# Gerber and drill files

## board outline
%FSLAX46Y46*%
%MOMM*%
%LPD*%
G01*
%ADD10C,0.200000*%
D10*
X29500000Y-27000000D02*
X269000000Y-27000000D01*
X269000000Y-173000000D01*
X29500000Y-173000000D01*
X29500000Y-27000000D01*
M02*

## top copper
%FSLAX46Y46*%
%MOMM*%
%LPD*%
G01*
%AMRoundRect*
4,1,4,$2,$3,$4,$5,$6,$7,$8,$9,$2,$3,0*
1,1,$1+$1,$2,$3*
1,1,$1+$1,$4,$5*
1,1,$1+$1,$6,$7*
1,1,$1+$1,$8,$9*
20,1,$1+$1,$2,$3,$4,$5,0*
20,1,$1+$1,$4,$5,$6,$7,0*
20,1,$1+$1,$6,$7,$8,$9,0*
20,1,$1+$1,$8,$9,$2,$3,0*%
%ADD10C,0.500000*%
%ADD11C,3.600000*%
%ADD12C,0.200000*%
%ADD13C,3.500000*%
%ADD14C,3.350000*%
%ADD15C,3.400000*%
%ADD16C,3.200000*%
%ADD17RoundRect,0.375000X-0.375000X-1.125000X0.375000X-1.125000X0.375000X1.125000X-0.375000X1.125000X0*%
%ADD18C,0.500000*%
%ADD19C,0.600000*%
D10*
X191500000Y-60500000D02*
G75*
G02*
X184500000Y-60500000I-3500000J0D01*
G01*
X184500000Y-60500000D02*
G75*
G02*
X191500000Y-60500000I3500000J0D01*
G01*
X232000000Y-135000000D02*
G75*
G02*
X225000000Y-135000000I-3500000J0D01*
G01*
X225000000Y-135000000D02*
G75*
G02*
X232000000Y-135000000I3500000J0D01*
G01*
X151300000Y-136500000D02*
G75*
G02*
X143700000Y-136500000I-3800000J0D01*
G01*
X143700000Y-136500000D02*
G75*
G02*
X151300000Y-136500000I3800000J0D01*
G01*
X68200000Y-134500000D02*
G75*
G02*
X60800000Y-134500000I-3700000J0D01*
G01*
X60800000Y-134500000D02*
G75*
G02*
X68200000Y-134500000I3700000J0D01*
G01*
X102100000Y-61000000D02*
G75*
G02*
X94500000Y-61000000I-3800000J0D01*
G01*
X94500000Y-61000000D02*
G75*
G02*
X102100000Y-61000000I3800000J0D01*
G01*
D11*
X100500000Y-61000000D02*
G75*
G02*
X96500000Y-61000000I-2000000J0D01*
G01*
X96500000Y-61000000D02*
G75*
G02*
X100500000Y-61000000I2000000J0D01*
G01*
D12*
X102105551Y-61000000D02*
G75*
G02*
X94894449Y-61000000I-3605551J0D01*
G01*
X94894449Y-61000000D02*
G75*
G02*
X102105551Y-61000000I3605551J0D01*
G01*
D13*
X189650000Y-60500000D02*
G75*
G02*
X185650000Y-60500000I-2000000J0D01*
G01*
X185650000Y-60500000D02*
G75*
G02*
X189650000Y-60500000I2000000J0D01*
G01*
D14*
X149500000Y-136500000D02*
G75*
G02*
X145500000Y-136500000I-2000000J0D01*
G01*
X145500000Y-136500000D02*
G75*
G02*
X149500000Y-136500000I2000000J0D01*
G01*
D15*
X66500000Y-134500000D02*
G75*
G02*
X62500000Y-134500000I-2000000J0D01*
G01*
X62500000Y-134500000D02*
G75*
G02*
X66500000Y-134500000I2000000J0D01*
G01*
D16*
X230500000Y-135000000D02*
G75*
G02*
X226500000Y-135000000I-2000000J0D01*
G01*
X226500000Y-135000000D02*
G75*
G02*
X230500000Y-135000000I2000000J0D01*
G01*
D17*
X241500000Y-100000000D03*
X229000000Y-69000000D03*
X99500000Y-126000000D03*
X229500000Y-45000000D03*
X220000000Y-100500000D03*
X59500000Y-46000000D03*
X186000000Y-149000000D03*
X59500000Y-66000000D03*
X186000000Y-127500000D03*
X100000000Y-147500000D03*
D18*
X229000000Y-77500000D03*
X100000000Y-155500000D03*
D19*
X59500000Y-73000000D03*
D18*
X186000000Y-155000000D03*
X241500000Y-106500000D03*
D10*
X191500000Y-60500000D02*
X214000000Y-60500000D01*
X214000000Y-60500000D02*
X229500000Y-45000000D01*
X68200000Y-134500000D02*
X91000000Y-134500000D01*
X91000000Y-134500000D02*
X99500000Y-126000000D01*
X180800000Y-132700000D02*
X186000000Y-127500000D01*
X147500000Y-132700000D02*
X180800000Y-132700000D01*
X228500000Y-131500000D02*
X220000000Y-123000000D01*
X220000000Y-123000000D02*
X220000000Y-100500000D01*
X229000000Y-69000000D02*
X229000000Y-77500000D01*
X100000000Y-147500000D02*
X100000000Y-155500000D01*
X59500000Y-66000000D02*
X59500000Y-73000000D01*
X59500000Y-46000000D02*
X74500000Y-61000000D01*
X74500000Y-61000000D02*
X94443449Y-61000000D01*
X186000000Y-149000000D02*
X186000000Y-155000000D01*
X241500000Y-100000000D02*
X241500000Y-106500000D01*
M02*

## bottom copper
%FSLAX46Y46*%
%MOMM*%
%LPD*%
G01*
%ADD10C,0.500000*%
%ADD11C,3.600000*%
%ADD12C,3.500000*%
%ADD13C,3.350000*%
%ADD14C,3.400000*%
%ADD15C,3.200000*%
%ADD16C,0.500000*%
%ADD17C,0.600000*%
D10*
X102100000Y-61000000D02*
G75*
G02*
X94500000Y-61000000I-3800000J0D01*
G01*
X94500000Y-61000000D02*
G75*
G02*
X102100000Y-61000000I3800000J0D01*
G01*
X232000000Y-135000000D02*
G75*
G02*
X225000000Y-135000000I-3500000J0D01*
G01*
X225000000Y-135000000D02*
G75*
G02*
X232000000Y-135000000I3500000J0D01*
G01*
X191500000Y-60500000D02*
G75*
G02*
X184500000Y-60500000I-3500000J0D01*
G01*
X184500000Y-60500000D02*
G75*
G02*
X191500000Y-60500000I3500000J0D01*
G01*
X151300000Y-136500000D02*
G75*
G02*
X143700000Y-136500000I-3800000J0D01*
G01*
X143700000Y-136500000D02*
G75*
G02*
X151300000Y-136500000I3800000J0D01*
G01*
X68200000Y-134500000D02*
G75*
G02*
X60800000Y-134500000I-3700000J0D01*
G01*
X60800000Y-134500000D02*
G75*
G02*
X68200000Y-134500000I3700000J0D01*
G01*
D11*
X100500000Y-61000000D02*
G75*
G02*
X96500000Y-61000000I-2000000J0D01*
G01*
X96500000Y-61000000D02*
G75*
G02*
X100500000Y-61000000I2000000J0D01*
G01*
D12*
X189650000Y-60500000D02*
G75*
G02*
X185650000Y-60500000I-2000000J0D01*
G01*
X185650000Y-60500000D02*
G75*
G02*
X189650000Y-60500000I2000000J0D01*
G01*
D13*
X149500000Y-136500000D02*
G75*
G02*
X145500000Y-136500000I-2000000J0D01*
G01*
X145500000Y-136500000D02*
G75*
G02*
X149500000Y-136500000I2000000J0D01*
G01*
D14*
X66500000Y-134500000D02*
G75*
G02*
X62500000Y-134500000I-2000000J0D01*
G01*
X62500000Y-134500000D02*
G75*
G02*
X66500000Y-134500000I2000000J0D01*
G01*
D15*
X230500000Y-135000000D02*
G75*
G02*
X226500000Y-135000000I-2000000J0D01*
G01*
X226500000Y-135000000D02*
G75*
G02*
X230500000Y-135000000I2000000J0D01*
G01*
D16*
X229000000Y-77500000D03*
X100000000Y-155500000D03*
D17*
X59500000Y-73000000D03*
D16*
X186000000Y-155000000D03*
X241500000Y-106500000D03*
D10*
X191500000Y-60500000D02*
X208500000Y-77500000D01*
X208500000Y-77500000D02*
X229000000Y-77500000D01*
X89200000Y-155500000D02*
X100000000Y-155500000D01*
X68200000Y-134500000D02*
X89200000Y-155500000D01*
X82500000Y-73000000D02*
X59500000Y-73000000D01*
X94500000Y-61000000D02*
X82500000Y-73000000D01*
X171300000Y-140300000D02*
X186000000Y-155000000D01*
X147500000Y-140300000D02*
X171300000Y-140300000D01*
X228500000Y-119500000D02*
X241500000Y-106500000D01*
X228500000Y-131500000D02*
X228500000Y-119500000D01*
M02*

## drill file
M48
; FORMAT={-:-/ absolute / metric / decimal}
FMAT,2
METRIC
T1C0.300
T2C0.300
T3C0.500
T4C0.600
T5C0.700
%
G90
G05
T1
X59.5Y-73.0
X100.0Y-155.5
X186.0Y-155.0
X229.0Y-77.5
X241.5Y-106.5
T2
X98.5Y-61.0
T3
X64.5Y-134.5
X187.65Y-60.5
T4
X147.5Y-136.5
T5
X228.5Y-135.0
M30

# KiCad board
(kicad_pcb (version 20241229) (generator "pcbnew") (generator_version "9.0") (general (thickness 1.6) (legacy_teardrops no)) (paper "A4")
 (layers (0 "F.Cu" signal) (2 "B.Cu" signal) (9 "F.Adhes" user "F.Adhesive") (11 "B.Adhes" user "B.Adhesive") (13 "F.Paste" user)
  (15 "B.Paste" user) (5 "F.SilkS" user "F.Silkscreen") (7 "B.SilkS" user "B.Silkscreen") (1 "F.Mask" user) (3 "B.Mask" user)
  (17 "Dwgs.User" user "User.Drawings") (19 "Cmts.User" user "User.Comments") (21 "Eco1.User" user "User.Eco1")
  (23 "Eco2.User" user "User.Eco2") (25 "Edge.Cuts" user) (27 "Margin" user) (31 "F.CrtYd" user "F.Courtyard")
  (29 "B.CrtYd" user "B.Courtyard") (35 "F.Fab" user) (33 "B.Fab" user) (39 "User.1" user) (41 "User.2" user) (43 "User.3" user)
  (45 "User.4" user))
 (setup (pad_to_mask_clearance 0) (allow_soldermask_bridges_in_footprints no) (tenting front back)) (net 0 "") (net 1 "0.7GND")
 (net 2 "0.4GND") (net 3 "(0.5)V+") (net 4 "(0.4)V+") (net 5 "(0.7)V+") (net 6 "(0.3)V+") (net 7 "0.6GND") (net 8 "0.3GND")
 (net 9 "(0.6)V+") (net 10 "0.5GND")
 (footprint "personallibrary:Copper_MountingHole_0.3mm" (layer "F.Cu") (at 98.5 61.5)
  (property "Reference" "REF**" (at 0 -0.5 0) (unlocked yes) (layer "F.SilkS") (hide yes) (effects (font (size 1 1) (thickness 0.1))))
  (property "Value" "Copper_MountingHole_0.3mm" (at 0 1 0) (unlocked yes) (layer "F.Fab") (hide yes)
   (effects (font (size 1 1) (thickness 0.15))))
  (fp_circle (center 0 -0.5) (end 2 -0.5) (stroke (width 3.6) (type solid)) (fill no) (layers "F.Cu" "F.Mask"))
  (fp_circle (center 0 -0.5) (end 3 -2.5) (stroke (width 0.2) (type solid)) (fill no) (layer "F.Cu"))
  (fp_circle (center 0 -0.5) (end 2 -0.5) (stroke (width 3.6) (type solid)) (fill no) (layers "B.Cu" "B.Mask"))
  (pad "" np_thru_hole circle (at 0 -0.5) (size 0.3 0.3) (drill 0.3) (layers "*.Cu" "*.Mask")))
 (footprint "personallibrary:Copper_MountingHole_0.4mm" (layer "F.Cu") (at 187.5 60.5)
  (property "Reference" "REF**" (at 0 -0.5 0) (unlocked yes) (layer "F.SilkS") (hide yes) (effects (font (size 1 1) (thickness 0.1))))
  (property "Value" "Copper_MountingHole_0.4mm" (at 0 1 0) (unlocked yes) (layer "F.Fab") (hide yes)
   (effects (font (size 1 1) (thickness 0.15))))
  (fp_circle (center 0.15 0) (end 2.15 0) (stroke (width 3.5) (type solid)) (fill no) (layers "F.Cu" "F.Mask"))
  (fp_circle (center 0.15 0) (end 2.15 0) (stroke (width 3.5) (type solid)) (fill no) (layers "B.Cu" "B.Mask"))
  (pad "" np_thru_hole circle (at 0.15 0) (size 0.5 0.5) (drill 0.5) (layers "*.Cu" "*.Mask")))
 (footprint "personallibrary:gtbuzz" (layer "F.Cu") (at 47 91.5)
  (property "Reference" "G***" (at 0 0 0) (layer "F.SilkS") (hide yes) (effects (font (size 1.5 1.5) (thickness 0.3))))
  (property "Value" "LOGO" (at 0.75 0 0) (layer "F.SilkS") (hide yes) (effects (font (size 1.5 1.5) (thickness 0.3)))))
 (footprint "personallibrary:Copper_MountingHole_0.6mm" (layer "F.Cu") (at 147.5 137)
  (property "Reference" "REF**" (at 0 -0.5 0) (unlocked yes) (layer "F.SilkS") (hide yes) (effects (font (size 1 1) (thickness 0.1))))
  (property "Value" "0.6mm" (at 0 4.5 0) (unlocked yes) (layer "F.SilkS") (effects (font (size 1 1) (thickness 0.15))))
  (fp_circle (center 0 -0.5) (end 2 -0.5) (stroke (width 3.35) (type solid)) (fill no) (layers "F.Cu" "F.Mask"))
  (fp_circle (center 0 -0.5) (end 2 -0.5) (stroke (width 3.35) (type solid)) (fill no) (layers "B.Cu" "B.Mask"))
  (pad "" np_thru_hole circle (at 0 -0.5) (size 0.6 0.6) (drill 0.6) (layers "*.Cu" "*.Mask")))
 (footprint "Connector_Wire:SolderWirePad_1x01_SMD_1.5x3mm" (layer "F.Cu") (at 241.5 100)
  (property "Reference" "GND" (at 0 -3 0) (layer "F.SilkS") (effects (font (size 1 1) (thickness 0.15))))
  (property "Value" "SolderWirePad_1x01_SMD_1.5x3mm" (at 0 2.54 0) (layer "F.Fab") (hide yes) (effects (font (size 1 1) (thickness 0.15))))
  (pad "9" smd roundrect (at 0 0) (size 1.5 3) (layers "F.Cu" "F.Mask") (roundrect_rratio 0.25) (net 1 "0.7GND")))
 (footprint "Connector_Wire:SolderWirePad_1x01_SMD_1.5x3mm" (layer "F.Cu") (at 229 69)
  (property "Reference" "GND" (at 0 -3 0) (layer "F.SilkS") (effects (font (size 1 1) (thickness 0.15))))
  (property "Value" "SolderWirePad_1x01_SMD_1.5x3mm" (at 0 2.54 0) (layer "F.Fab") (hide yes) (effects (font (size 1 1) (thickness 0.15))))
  (pad "7" smd roundrect (at 0 0) (size 1.5 3) (layers "F.Cu" "F.Mask") (roundrect_rratio 0.25) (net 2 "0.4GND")))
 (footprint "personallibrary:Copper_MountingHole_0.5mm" (layer "F.Cu") (at 64.35 134.5)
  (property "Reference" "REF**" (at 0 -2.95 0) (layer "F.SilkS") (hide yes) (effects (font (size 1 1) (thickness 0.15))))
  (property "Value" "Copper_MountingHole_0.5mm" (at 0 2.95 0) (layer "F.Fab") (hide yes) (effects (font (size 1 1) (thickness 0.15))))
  (fp_circle (center 0.15 0) (end 2.15 0) (stroke (width 3.4) (type solid)) (fill no) (layers "F.Cu" "F.Mask"))
  (fp_circle (center 0.15 0) (end 2.15 0) (stroke (width 3.4) (type solid)) (fill no) (layers "B.Cu" "B.Mask"))
  (pad "" np_thru_hole circle (at 0.15 0) (size 0.5 0.5) (drill 0.5) (layers "*.Cu" "*.Mask")))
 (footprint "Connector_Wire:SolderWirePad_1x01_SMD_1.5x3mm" (layer "F.Cu") (at 99.5 126)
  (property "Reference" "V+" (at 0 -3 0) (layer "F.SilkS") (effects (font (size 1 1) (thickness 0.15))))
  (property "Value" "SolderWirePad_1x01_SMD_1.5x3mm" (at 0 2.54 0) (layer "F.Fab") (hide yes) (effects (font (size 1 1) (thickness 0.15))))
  (pad "4" smd roundrect (at 0 0) (size 1.5 3) (layers "F.Cu" "F.Mask") (roundrect_rratio 0.25) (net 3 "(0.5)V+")))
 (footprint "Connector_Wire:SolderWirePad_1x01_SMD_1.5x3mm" (layer "F.Cu") (at 229.5 45)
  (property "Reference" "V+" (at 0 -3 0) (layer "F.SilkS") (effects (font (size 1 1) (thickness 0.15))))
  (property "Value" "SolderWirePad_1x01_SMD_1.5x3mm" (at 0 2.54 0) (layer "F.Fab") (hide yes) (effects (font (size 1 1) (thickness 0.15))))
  (pad "3" smd roundrect (at 0 0) (size 1.5 3) (layers "F.Cu" "F.Mask") (roundrect_rratio 0.25) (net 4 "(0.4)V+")))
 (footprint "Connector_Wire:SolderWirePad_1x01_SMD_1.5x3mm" (layer "F.Cu") (at 220 100.5)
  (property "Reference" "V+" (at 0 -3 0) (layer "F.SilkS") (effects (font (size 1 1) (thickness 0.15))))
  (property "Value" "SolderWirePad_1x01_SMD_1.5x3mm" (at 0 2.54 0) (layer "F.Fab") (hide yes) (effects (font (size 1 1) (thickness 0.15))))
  (pad "6" smd roundrect (at 0 0) (size 1.5 3) (layers "F.Cu" "F.Mask") (roundrect_rratio 0.25) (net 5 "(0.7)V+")))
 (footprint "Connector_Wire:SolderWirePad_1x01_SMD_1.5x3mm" (layer "F.Cu") (at 59.5 46)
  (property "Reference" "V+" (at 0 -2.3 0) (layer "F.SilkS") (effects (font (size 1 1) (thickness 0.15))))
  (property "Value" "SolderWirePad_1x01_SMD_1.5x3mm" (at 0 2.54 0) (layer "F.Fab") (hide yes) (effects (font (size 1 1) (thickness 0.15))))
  (pad "1" smd roundrect (at 0 0) (size 1.5 3) (layers "F.Cu" "F.Mask") (roundrect_rratio 0.25) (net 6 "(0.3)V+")))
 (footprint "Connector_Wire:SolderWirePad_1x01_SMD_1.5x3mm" (layer "F.Cu") (at 186 149)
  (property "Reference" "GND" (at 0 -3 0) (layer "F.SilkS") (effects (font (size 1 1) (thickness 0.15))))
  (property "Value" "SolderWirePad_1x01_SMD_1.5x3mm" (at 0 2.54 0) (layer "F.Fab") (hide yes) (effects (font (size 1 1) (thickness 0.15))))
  (pad "9" smd roundrect (at 0 0) (size 1.5 3) (layers "F.Cu" "F.Mask") (roundrect_rratio 0.25) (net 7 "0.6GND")))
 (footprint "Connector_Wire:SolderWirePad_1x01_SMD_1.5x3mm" (layer "F.Cu") (at 59.5 66)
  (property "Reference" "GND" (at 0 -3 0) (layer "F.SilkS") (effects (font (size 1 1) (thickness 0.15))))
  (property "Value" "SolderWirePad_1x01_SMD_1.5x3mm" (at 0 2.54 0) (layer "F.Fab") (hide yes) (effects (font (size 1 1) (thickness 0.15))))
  (pad "2" smd roundrect (at 0 0) (size 1.5 3) (layers "F.Cu" "F.Mask") (roundrect_rratio 0.25) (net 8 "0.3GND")))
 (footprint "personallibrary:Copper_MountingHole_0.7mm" (layer "F.Cu") (at 228.5 135.5)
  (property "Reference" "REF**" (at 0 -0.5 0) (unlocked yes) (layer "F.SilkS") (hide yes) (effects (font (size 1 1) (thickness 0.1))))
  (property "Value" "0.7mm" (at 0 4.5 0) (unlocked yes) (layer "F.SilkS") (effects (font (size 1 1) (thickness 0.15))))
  (fp_circle (center 0 -0.5) (end 2 -0.5) (stroke (width 3.2) (type solid)) (fill no) (layers "F.Cu" "F.Mask"))
  (fp_circle (center 0 -0.5) (end 2 -0.5) (stroke (width 3.2) (type solid)) (fill no) (layers "B.Cu" "B.Mask"))
  (pad "" np_thru_hole circle (at 0 -0.5) (size 0.7 0.7) (drill 0.7) (layers "*.Cu" "*.Mask")))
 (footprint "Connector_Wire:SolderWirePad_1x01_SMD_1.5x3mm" (layer "F.Cu") (at 186 127.5)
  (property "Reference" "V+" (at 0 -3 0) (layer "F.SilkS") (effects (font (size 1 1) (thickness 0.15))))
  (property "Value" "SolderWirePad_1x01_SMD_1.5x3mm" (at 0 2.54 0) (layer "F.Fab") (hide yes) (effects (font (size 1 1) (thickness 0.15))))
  (pad "5" smd roundrect (at 0 0) (size 1.5 3) (layers "F.Cu" "F.Mask") (roundrect_rratio 0.25) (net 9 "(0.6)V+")))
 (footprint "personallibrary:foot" (layer "F.Cu") (at 43.5 51.5)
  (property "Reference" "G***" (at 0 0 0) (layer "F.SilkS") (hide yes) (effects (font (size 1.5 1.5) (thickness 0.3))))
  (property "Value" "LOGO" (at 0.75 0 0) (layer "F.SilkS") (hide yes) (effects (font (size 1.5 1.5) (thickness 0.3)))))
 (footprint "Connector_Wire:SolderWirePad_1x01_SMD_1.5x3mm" (layer "F.Cu") (at 100 147.5)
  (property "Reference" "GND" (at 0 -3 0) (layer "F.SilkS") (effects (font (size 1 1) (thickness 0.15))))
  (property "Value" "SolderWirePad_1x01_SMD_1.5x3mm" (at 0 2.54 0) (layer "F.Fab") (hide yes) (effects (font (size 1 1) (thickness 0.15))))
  (pad "8" smd roundrect (at 0 0) (size 1.5 3) (layers "F.Cu" "F.Mask") (roundrect_rratio 0.25) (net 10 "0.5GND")))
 (gr_circle (center 188 60.5) (end 184.5 60.5) (stroke (width 0.5) (type solid)) (fill no) (layer "F.Cu") (net 4))
 (gr_circle (center 228.5 135) (end 232 135) (stroke (width 0.5) (type solid)) (fill no) (layer "F.Cu") (net 5))
 (gr_circle (center 147.5 136.5) (end 151.3 136.5) (stroke (width 0.5) (type solid)) (fill no) (layer "F.Cu") (net 9))
 (gr_circle (center 64.5 134.5) (end 68.2 134.5) (stroke (width 0.5) (type solid)) (fill no) (layer "F.Cu") (net 3))
 (gr_circle (center 98.3 61) (end 102.1 61) (stroke (width 0.5) (type solid)) (fill no) (layer "F.Cu") (net 6))
 (gr_circle (center 98.3 61) (end 102.1 61) (stroke (width 0.5) (type solid)) (fill no) (layer "B.Cu") (net 8))
 (gr_circle (center 228.5 135) (end 232 135) (stroke (width 0.5) (type solid)) (fill no) (layer "B.Cu") (net 1))
 (gr_circle (center 188 60.5) (end 184.5 60.5) (stroke (width 0.5) (type solid)) (fill no) (layer "B.Cu") (net 2))
 (gr_circle (center 147.5 136.5) (end 151.3 136.5) (stroke (width 0.5) (type solid)) (fill no) (layer "B.Cu") (net 7))
 (gr_circle (center 64.5 134.5) (end 68.2 134.5) (stroke (width 0.5) (type solid)) (fill no) (layer "B.Cu") (net 10))
 (gr_rect (start 29.5 27) (end 269 173) (stroke (width 0.2) (type solid)) (fill no) (layer "Edge.Cuts"))
 (segment (start 191.5 60.5) (end 214 60.5) (width 0.5) (layer "F.Cu") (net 4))
 (segment (start 214 60.5) (end 229.5 45) (width 0.5) (layer "F.Cu") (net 4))
 (segment (start 68.2 134.5) (end 91 134.5) (width 0.5) (layer "F.Cu") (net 3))
 (segment (start 91 134.5) (end 99.5 126) (width 0.5) (layer "F.Cu") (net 3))
 (segment (start 180.8 132.7) (end 186 127.5) (width 0.5) (layer "F.Cu") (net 9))
 (segment (start 147.5 132.7) (end 180.8 132.7) (width 0.5) (layer "F.Cu") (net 9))
 (segment (start 228.5 131.5) (end 220 123) (width 0.5) (layer "F.Cu") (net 5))
 (segment (start 220 123) (end 220 100.5) (width 0.5) (layer "F.Cu") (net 5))
 (segment (start 229 69) (end 229 77.5) (width 0.5) (layer "F.Cu") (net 2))
 (via (at 229 77.5) (size 0.5) (drill 0.3) (layers "F.Cu" "B.Cu") (free yes) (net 2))
 (segment (start 191.5 60.5) (end 208.5 77.5) (width 0.5) (layer "B.Cu") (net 2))
 (segment (start 208.5 77.5) (end 229 77.5) (width 0.5) (layer "B.Cu") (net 2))
 (segment (start 100 147.5) (end 100 155.5) (width 0.5) (layer "F.Cu") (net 10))
 (via (at 100 155.5) (size 0.5) (drill 0.3) (layers "F.Cu" "B.Cu") (free yes) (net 10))
 (segment (start 89.2 155.5) (end 100 155.5) (width 0.5) (layer "B.Cu") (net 10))
 (segment (start 68.2 134.5) (end 89.2 155.5) (width 0.5) (layer "B.Cu") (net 10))
 (segment (start 59.5 66) (end 59.5 73) (width 0.5) (layer "F.Cu") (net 8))
 (via (at 59.5 73) (size 0.6) (drill 0.3) (layers "F.Cu" "B.Cu") (free yes) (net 8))
 (segment (start 82.5 73) (end 59.5 73) (width 0.5) (layer "B.Cu") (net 8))
 (segment (start 94.5 61) (end 82.5 73) (width 0.5) (layer "B.Cu") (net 8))
 (segment (start 59.5 46) (end 74.5 61) (width 0.5) (layer "F.Cu") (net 6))
 (segment (start 74.5 61) (end 94.443449 61) (width 0.5) (layer "F.Cu") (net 6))
 (segment (start 186 149) (end 186 155) (width 0.5) (layer "F.Cu") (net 7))
 (via (at 186 155) (size 0.5) (drill 0.3) (layers "F.Cu" "B.Cu") (free yes) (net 7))
 (segment (start 171.3 140.3) (end 186 155) (width 0.5) (layer "B.Cu") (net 7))
 (segment (start 147.5 140.3) (end 171.3 140.3) (width 0.5) (layer "B.Cu") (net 7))
 (segment (start 241.5 100) (end 241.5 106.5) (width 0.5) (layer "F.Cu") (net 1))
 (via (at 241.5 106.5) (size 0.5) (drill 0.3) (layers "F.Cu" "B.Cu") (free yes) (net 1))
 (segment (start 228.5 119.5) (end 241.5 106.5) (width 0.5) (layer "B.Cu") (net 1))
 (segment (start 228.5 131.5) (end 228.5 119.5) (width 0.5) (layer "B.Cu") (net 1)))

